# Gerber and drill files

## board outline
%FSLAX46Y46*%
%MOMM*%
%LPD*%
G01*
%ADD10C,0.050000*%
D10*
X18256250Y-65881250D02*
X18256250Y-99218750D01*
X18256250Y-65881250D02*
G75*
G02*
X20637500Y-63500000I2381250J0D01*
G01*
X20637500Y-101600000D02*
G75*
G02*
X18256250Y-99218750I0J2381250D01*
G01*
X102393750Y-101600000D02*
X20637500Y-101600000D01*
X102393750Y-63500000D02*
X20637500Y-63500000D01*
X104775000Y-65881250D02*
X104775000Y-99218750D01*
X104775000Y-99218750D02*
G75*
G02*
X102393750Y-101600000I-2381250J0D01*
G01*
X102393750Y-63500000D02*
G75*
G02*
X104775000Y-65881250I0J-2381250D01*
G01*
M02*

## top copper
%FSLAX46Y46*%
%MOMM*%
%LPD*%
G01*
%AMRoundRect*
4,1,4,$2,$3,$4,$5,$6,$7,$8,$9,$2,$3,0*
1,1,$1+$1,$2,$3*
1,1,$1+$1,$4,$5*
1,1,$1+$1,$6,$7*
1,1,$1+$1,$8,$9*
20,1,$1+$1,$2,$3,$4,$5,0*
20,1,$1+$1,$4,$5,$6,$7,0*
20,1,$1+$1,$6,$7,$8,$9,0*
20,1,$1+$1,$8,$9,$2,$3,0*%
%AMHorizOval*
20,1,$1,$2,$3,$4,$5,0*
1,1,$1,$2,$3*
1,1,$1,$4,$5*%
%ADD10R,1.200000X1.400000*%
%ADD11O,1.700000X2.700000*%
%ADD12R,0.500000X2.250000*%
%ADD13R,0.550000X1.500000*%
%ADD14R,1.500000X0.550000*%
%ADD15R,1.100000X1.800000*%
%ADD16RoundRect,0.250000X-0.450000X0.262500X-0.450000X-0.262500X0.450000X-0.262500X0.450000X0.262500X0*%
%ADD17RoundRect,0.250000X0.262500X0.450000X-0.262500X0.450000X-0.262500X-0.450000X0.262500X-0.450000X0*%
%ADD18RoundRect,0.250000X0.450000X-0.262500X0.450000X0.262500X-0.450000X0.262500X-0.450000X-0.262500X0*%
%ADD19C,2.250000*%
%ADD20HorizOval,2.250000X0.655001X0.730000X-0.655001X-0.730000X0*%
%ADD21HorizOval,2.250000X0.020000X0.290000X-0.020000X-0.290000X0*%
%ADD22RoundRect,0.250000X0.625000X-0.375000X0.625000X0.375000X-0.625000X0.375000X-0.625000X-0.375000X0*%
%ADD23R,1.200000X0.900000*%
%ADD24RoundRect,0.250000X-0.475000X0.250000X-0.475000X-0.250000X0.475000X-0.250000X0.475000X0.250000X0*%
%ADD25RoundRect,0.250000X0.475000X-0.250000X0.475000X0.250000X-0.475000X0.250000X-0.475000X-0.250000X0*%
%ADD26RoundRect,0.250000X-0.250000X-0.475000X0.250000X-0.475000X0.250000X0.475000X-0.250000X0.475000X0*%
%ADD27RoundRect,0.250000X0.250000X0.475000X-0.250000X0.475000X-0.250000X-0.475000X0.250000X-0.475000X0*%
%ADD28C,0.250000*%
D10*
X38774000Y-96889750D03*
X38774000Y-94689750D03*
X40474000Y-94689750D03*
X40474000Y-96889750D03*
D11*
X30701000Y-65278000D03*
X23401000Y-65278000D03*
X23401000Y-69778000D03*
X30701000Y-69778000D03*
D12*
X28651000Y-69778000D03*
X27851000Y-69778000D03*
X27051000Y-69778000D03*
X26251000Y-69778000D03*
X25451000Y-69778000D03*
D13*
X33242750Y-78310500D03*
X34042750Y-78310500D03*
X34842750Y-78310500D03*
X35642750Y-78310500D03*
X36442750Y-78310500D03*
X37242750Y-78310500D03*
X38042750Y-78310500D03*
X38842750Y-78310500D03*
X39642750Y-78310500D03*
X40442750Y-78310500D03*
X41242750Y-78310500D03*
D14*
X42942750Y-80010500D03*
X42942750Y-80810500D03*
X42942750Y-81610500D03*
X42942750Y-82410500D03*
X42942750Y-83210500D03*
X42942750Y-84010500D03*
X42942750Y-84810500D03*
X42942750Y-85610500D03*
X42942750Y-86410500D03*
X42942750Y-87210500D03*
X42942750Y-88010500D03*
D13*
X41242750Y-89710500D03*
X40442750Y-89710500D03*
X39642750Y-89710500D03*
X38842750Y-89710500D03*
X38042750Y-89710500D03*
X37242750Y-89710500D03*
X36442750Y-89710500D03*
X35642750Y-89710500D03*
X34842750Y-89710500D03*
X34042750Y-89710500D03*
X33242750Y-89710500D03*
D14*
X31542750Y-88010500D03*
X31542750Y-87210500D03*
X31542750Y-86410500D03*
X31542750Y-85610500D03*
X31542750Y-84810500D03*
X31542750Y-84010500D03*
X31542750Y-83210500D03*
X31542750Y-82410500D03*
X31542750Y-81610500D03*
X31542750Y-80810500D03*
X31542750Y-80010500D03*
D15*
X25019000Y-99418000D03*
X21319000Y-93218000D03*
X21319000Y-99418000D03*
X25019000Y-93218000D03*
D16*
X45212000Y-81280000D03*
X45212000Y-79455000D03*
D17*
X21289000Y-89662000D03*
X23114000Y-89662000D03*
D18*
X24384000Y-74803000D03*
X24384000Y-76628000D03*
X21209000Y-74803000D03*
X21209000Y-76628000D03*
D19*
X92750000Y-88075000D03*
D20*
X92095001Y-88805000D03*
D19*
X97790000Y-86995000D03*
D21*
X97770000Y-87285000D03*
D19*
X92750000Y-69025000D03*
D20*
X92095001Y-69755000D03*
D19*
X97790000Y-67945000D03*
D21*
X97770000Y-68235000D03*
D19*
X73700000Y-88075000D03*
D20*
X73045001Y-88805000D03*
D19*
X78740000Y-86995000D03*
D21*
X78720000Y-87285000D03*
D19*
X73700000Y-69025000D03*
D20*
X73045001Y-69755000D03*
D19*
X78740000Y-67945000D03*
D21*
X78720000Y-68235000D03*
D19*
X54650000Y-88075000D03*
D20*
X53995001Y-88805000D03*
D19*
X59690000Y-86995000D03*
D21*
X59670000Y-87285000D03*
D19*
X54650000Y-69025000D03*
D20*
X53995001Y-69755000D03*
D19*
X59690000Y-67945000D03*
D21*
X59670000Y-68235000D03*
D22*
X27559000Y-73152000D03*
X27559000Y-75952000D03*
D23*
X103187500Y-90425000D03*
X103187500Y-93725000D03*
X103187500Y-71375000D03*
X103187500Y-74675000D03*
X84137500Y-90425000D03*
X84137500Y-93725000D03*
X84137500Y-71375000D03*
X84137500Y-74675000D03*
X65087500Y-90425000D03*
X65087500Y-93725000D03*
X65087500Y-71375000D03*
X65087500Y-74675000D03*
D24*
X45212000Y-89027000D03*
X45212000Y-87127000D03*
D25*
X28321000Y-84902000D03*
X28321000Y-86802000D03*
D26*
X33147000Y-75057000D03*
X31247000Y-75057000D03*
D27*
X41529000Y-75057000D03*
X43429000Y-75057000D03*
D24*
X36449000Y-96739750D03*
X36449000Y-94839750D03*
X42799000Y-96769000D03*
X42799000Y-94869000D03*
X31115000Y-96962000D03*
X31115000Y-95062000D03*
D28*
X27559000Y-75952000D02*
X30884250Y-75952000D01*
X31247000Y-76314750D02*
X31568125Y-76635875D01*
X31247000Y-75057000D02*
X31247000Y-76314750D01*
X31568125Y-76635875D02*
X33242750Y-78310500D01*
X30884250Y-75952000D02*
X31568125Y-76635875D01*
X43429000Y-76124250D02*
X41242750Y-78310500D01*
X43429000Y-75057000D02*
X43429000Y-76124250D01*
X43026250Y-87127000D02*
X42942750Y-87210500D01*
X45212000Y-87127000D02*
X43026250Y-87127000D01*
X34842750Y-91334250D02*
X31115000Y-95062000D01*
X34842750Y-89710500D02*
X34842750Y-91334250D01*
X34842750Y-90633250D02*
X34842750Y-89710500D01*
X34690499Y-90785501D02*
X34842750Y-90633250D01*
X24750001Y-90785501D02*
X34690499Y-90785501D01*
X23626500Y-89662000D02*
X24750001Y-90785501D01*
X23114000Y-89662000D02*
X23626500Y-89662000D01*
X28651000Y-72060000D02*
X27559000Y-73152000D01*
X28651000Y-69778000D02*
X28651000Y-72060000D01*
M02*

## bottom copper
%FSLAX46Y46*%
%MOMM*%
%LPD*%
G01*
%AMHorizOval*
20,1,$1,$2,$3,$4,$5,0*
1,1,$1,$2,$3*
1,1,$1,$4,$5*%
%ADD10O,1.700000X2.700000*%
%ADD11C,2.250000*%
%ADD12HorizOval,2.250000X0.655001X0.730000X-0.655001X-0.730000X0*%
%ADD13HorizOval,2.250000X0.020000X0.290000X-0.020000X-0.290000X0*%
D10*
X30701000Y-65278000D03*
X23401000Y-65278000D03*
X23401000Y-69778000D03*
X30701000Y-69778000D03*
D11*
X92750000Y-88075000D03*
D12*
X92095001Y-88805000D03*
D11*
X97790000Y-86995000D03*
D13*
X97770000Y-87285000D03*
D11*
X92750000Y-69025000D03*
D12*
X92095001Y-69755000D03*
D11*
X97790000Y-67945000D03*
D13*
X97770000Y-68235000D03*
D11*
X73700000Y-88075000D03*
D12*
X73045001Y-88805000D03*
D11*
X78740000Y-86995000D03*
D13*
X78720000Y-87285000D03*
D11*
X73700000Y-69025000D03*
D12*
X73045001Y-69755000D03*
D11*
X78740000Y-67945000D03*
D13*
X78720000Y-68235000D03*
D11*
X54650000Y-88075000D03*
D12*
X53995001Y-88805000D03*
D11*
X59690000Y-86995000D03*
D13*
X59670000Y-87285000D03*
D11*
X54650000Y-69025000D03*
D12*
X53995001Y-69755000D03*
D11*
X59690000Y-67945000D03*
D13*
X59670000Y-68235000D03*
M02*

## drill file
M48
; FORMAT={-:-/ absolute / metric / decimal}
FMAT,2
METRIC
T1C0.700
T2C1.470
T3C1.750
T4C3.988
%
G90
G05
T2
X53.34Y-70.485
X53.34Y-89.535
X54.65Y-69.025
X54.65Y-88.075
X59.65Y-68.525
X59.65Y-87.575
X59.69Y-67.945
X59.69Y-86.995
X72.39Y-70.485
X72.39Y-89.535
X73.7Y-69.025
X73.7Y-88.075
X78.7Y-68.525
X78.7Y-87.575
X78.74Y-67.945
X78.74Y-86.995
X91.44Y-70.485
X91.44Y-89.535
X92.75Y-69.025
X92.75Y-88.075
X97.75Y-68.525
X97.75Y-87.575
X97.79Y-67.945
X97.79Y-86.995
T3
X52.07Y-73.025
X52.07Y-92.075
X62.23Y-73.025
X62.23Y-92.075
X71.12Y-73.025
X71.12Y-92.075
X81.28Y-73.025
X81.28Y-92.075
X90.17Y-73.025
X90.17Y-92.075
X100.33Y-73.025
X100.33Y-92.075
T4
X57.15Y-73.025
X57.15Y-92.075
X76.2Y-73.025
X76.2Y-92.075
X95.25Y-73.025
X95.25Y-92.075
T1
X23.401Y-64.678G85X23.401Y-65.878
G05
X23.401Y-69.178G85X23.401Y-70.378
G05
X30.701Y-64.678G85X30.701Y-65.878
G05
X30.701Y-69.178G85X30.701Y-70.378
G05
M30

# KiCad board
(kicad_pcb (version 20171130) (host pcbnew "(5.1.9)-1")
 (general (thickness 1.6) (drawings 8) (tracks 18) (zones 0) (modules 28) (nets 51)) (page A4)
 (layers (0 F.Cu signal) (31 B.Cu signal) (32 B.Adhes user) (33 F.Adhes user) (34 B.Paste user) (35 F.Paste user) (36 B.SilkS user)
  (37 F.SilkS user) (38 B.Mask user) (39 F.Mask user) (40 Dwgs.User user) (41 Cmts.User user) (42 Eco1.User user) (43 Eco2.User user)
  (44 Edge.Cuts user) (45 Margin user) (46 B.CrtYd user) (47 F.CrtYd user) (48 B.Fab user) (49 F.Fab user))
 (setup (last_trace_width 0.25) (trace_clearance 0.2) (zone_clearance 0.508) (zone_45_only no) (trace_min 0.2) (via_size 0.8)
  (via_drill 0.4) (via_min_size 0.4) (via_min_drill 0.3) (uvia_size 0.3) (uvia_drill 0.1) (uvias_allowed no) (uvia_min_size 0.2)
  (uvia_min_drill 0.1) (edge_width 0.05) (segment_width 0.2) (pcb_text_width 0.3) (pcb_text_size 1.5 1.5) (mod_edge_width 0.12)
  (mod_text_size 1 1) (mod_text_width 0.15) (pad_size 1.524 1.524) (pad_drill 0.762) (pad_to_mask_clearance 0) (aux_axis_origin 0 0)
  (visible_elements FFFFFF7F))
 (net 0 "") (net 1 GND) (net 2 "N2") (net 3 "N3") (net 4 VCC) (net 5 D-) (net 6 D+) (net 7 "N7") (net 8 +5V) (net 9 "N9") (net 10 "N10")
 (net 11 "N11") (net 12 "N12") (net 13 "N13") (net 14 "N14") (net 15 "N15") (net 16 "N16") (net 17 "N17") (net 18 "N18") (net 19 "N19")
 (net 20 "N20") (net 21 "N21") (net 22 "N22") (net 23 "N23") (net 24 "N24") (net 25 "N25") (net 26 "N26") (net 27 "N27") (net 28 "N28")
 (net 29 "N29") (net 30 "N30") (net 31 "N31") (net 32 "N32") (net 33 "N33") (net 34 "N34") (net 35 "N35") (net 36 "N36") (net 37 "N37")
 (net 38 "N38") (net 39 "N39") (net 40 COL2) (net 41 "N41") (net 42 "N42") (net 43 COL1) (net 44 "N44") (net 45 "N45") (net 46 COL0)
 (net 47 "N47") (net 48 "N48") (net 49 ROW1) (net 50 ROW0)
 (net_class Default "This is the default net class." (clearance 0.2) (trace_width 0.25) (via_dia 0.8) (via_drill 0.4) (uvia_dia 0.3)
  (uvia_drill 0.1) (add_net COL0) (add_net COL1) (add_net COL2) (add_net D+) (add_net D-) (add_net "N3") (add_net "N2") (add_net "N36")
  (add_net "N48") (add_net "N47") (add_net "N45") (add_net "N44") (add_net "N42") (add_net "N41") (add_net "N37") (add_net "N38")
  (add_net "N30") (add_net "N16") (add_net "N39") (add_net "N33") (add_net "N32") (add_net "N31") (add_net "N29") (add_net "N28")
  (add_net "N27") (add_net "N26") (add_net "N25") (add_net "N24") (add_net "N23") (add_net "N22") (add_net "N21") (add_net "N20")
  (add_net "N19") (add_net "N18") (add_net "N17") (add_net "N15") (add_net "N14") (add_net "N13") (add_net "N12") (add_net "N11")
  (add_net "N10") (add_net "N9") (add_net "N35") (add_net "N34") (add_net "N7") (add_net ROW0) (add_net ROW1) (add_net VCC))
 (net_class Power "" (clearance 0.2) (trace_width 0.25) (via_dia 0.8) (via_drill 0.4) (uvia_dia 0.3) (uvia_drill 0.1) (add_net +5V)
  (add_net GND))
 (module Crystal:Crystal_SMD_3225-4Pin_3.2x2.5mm (layer F.Cu) (at 39.624 95.78975 90)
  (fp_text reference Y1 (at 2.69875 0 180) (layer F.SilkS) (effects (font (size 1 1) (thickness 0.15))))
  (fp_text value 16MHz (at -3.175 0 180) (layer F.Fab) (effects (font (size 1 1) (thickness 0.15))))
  (pad 4 smd rect (at -1.1 -0.85 90) (size 1.4 1.2) (layers F.Cu F.Paste F.Mask) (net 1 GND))
  (pad 3 smd rect (at 1.1 -0.85 90) (size 1.4 1.2) (layers F.Cu F.Paste F.Mask) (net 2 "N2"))
  (pad 2 smd rect (at 1.1 0.85 90) (size 1.4 1.2) (layers F.Cu F.Paste F.Mask) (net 1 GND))
  (pad 1 smd rect (at -1.1 0.85 90) (size 1.4 1.2) (layers F.Cu F.Paste F.Mask) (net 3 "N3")))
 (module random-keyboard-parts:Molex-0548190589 (layer F.Cu) (at 27.051 65.278 270)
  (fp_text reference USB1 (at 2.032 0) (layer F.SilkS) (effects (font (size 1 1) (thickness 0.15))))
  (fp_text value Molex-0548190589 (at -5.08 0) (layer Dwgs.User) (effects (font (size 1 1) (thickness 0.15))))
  (pad 6 thru_hole oval (at 0 -3.65 270) (size 2.7 1.7) (drill oval 1.9 0.7) (layers *.Cu *.Mask) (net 1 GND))
  (pad 6 thru_hole oval (at 0 3.65 270) (size 2.7 1.7) (drill oval 1.9 0.7) (layers *.Cu *.Mask) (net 1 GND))
  (pad 6 thru_hole oval (at 4.5 3.65 270) (size 2.7 1.7) (drill oval 1.9 0.7) (layers *.Cu *.Mask) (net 1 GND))
  (pad 6 thru_hole oval (at 4.5 -3.65 270) (size 2.7 1.7) (drill oval 1.9 0.7) (layers *.Cu *.Mask) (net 1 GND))
  (pad 5 smd rect (at 4.5 -1.6 270) (size 2.25 0.5) (layers F.Cu F.Paste F.Mask) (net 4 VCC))
  (pad 4 smd rect (at 4.5 -0.8 270) (size 2.25 0.5) (layers F.Cu F.Paste F.Mask) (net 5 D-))
  (pad 3 smd rect (at 4.5 0 270) (size 2.25 0.5) (layers F.Cu F.Paste F.Mask) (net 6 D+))
  (pad 2 smd rect (at 4.5 0.8 270) (size 2.25 0.5) (layers F.Cu F.Paste F.Mask) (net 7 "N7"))
  (pad 1 smd rect (at 4.5 1.6 270) (size 2.25 0.5) (layers F.Cu F.Paste F.Mask) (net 1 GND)))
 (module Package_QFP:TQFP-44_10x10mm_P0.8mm (layer F.Cu) (at 37.24275 84.0105)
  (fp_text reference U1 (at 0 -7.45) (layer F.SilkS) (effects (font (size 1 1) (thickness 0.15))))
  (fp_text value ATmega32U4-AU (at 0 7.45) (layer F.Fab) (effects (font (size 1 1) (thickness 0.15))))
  (pad 44 smd rect (at -4 -5.7 90) (size 1.5 0.55) (layers F.Cu F.Paste F.Mask) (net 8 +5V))
  (pad 43 smd rect (at -3.2 -5.7 90) (size 1.5 0.55) (layers F.Cu F.Paste F.Mask) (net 1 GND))
  (pad 42 smd rect (at -2.4 -5.7 90) (size 1.5 0.55) (layers F.Cu F.Paste F.Mask) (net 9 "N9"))
  (pad 41 smd rect (at -1.6 -5.7 90) (size 1.5 0.55) (layers F.Cu F.Paste F.Mask) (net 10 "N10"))
  (pad 40 smd rect (at -0.8 -5.7 90) (size 1.5 0.55) (layers F.Cu F.Paste F.Mask) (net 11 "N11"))
  (pad 39 smd rect (at 0 -5.7 90) (size 1.5 0.55) (layers F.Cu F.Paste F.Mask) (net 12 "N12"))
  (pad 38 smd rect (at 0.8 -5.7 90) (size 1.5 0.55) (layers F.Cu F.Paste F.Mask) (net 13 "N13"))
  (pad 37 smd rect (at 1.6 -5.7 90) (size 1.5 0.55) (layers F.Cu F.Paste F.Mask) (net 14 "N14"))
  (pad 36 smd rect (at 2.4 -5.7 90) (size 1.5 0.55) (layers F.Cu F.Paste F.Mask) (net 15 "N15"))
  (pad 35 smd rect (at 3.2 -5.7 90) (size 1.5 0.55) (layers F.Cu F.Paste F.Mask) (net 1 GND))
  (pad 34 smd rect (at 4 -5.7 90) (size 1.5 0.55) (layers F.Cu F.Paste F.Mask) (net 8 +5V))
  (pad 33 smd rect (at 5.7 -4) (size 1.5 0.55) (layers F.Cu F.Paste F.Mask) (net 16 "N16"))
  (pad 32 smd rect (at 5.7 -3.2) (size 1.5 0.55) (layers F.Cu F.Paste F.Mask) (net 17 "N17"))
  (pad 31 smd rect (at 5.7 -2.4) (size 1.5 0.55) (layers F.Cu F.Paste F.Mask) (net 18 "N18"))
  (pad 30 smd rect (at 5.7 -1.6) (size 1.5 0.55) (layers F.Cu F.Paste F.Mask) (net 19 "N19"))
  (pad 29 smd rect (at 5.7 -0.8) (size 1.5 0.55) (layers F.Cu F.Paste F.Mask) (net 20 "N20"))
  (pad 28 smd rect (at 5.7 0) (size 1.5 0.55) (layers F.Cu F.Paste F.Mask) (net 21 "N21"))
  (pad 27 smd rect (at 5.7 0.8) (size 1.5 0.55) (layers F.Cu F.Paste F.Mask) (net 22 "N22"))
  (pad 26 smd rect (at 5.7 1.6) (size 1.5 0.55) (layers F.Cu F.Paste F.Mask) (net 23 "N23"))
  (pad 25 smd rect (at 5.7 2.4) (size 1.5 0.55) (layers F.Cu F.Paste F.Mask) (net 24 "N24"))
  (pad 24 smd rect (at 5.7 3.2) (size 1.5 0.55) (layers F.Cu F.Paste F.Mask) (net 8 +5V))
  (pad 23 smd rect (at 5.7 4) (size 1.5 0.55) (layers F.Cu F.Paste F.Mask) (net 1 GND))
  (pad 22 smd rect (at 4 5.7 90) (size 1.5 0.55) (layers F.Cu F.Paste F.Mask) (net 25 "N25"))
  (pad 21 smd rect (at 3.2 5.7 90) (size 1.5 0.55) (layers F.Cu F.Paste F.Mask) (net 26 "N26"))
  (pad 20 smd rect (at 2.4 5.7 90) (size 1.5 0.55) (layers F.Cu F.Paste F.Mask) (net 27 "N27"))
  (pad 19 smd rect (at 1.6 5.7 90) (size 1.5 0.55) (layers F.Cu F.Paste F.Mask) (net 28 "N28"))
  (pad 18 smd rect (at 0.8 5.7 90) (size 1.5 0.55) (layers F.Cu F.Paste F.Mask) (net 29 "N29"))
  (pad 17 smd rect (at 0 5.7 90) (size 1.5 0.55) (layers F.Cu F.Paste F.Mask) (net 3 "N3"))
  (pad 16 smd rect (at -0.8 5.7 90) (size 1.5 0.55) (layers F.Cu F.Paste F.Mask) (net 2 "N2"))
  (pad 15 smd rect (at -1.6 5.7 90) (size 1.5 0.55) (layers F.Cu F.Paste F.Mask) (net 1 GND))
  (pad 14 smd rect (at -2.4 5.7 90) (size 1.5 0.55) (layers F.Cu F.Paste F.Mask) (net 8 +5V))
  (pad 13 smd rect (at -3.2 5.7 90) (size 1.5 0.55) (layers F.Cu F.Paste F.Mask) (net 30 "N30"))
  (pad 12 smd rect (at -4 5.7 90) (size 1.5 0.55) (layers F.Cu F.Paste F.Mask) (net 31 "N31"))
  (pad 11 smd rect (at -5.7 4) (size 1.5 0.55) (layers F.Cu F.Paste F.Mask) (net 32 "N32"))
  (pad 10 smd rect (at -5.7 3.2) (size 1.5 0.55) (layers F.Cu F.Paste F.Mask) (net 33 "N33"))
  (pad 9 smd rect (at -5.7 2.4) (size 1.5 0.55) (layers F.Cu F.Paste F.Mask) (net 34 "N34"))
  (pad 8 smd rect (at -5.7 1.6) (size 1.5 0.55) (layers F.Cu F.Paste F.Mask) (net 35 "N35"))
  (pad 7 smd rect (at -5.7 0.8) (size 1.5 0.55) (layers F.Cu F.Paste F.Mask) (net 8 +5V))
  (pad 6 smd rect (at -5.7 0) (size 1.5 0.55) (layers F.Cu F.Paste F.Mask) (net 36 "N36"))
  (pad 5 smd rect (at -5.7 -0.8) (size 1.5 0.55) (layers F.Cu F.Paste F.Mask) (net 1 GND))
  (pad 4 smd rect (at -5.7 -1.6) (size 1.5 0.55) (layers F.Cu F.Paste F.Mask) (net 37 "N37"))
  (pad 3 smd rect (at -5.7 -2.4) (size 1.5 0.55) (layers F.Cu F.Paste F.Mask) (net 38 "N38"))
  (pad 2 smd rect (at -5.7 -3.2) (size 1.5 0.55) (layers F.Cu F.Paste F.Mask) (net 8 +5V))
  (pad 1 smd rect (at -5.7 -4) (size 1.5 0.55) (layers F.Cu F.Paste F.Mask) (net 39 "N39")))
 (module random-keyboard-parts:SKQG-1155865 (layer F.Cu) (at 23.169 96.318 90)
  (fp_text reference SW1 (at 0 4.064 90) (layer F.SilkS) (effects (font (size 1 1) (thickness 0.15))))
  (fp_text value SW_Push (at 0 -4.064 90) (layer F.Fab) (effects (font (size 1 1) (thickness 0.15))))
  (pad 4 smd rect (at -3.1 1.85 90) (size 1.8 1.1) (layers F.Cu F.Paste F.Mask))
  (pad 3 smd rect (at 3.1 -1.85 90) (size 1.8 1.1) (layers F.Cu F.Paste F.Mask))
  (pad 2 smd rect (at -3.1 -1.85 90) (size 1.8 1.1) (layers F.Cu F.Paste F.Mask) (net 30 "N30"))
  (pad 1 smd rect (at 3.1 1.85 90) (size 1.8 1.1) (layers F.Cu F.Paste F.Mask) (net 1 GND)))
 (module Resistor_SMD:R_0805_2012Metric (layer F.Cu) (at 45.212 80.3675 270)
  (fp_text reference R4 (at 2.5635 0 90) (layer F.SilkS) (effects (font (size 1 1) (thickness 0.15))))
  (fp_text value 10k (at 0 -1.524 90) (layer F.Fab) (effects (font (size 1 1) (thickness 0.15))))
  (pad 2 smd roundrect (at 0.9125 0 270) (size 1.025 1.4) (layers F.Cu F.Paste F.Mask) (roundrect_rratio 0.243902) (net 16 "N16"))
  (pad 1 smd roundrect (at -0.9125 0 270) (size 1.025 1.4) (layers F.Cu F.Paste F.Mask) (roundrect_rratio 0.243902) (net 1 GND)))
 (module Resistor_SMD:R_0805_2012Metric (layer F.Cu) (at 22.2015 89.662 180)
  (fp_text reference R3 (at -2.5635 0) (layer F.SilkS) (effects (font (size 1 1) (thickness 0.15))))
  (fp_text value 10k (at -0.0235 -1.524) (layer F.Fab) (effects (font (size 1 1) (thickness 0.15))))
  (pad 2 smd roundrect (at 0.9125 0 180) (size 1.025 1.4) (layers F.Cu F.Paste F.Mask) (roundrect_rratio 0.243902) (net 30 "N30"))
  (pad 1 smd roundrect (at -0.9125 0 180) (size 1.025 1.4) (layers F.Cu F.Paste F.Mask) (roundrect_rratio 0.243902) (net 8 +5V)))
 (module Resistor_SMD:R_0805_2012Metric (layer F.Cu) (at 24.384 75.7155 90)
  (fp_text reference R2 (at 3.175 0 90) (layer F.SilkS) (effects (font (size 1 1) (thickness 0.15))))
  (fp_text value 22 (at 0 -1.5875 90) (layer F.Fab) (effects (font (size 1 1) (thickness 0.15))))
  (pad 2 smd roundrect (at 0.9125 0 90) (size 1.025 1.4) (layers F.Cu F.Paste F.Mask) (roundrect_rratio 0.243902) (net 5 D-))
  (pad 1 smd roundrect (at -0.9125 0 90) (size 1.025 1.4) (layers F.Cu F.Paste F.Mask) (roundrect_rratio 0.243902) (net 38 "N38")))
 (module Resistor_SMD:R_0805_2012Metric (layer F.Cu) (at 21.209 75.7155 90)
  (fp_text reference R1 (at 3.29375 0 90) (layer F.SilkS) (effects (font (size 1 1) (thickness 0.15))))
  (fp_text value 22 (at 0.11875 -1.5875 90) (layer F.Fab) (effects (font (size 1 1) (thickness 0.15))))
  (pad 2 smd roundrect (at 0.9125 0 90) (size 1.025 1.4) (layers F.Cu F.Paste F.Mask) (roundrect_rratio 0.243902) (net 6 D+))
  (pad 1 smd roundrect (at -0.9125 0 90) (size 1.025 1.4) (layers F.Cu F.Paste F.Mask) (roundrect_rratio 0.243902) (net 37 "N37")))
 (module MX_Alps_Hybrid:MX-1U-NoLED (layer F.Cu) (at 95.25 92.075)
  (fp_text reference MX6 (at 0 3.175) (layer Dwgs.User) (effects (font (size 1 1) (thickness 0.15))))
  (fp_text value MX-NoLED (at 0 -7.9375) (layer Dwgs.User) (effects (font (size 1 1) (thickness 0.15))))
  (pad "" np_thru_hole circle (at 5.08 0 48.0996) (size 1.75 1.75) (drill 1.75) (layers *.Cu *.Mask))
  (pad "" np_thru_hole circle (at -5.08 0 48.0996) (size 1.75 1.75) (drill 1.75) (layers *.Cu *.Mask))
  (pad 1 thru_hole circle (at -2.5 -4) (size 2.25 2.25) (drill 1.47) (layers *.Cu B.Mask) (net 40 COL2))
  (pad "" np_thru_hole circle (at 0 0) (size 3.9878 3.9878) (drill 3.9878) (layers *.Cu *.Mask))
  (pad 1 thru_hole oval (at -3.81 -2.54 48.0996) (size 4.211556 2.25) (drill 1.47 (offset 0.980778 0)) (layers *.Cu B.Mask) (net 40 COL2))
  (pad 2 thru_hole circle (at 2.54 -5.08) (size 2.25 2.25) (drill 1.47) (layers *.Cu B.Mask) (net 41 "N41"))
  (pad 2 thru_hole oval (at 2.5 -4.5 86.0548) (size 2.831378 2.25) (drill 1.47 (offset 0.290689 0)) (layers *.Cu B.Mask) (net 41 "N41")))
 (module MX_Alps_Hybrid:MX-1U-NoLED (layer F.Cu) (at 95.25 73.025)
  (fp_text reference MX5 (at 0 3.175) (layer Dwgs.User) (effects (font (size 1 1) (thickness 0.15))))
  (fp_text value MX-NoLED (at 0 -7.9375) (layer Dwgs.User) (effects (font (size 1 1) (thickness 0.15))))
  (pad "" np_thru_hole circle (at 5.08 0 48.0996) (size 1.75 1.75) (drill 1.75) (layers *.Cu *.Mask))
  (pad "" np_thru_hole circle (at -5.08 0 48.0996) (size 1.75 1.75) (drill 1.75) (layers *.Cu *.Mask))
  (pad 1 thru_hole circle (at -2.5 -4) (size 2.25 2.25) (drill 1.47) (layers *.Cu B.Mask) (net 40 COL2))
  (pad "" np_thru_hole circle (at 0 0) (size 3.9878 3.9878) (drill 3.9878) (layers *.Cu *.Mask))
  (pad 1 thru_hole oval (at -3.81 -2.54 48.0996) (size 4.211556 2.25) (drill 1.47 (offset 0.980778 0)) (layers *.Cu B.Mask) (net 40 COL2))
  (pad 2 thru_hole circle (at 2.54 -5.08) (size 2.25 2.25) (drill 1.47) (layers *.Cu B.Mask) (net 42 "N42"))
  (pad 2 thru_hole oval (at 2.5 -4.5 86.0548) (size 2.831378 2.25) (drill 1.47 (offset 0.290689 0)) (layers *.Cu B.Mask) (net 42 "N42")))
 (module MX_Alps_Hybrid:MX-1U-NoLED (layer F.Cu) (at 76.2 92.075)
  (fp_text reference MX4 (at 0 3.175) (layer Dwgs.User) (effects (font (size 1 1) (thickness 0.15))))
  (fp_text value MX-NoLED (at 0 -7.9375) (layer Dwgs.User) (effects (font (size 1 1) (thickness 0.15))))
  (pad "" np_thru_hole circle (at 5.08 0 48.0996) (size 1.75 1.75) (drill 1.75) (layers *.Cu *.Mask))
  (pad "" np_thru_hole circle (at -5.08 0 48.0996) (size 1.75 1.75) (drill 1.75) (layers *.Cu *.Mask))
  (pad 1 thru_hole circle (at -2.5 -4) (size 2.25 2.25) (drill 1.47) (layers *.Cu B.Mask) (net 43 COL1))
  (pad "" np_thru_hole circle (at 0 0) (size 3.9878 3.9878) (drill 3.9878) (layers *.Cu *.Mask))
  (pad 1 thru_hole oval (at -3.81 -2.54 48.0996) (size 4.211556 2.25) (drill 1.47 (offset 0.980778 0)) (layers *.Cu B.Mask) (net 43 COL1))
  (pad 2 thru_hole circle (at 2.54 -5.08) (size 2.25 2.25) (drill 1.47) (layers *.Cu B.Mask) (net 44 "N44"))
  (pad 2 thru_hole oval (at 2.5 -4.5 86.0548) (size 2.831378 2.25) (drill 1.47 (offset 0.290689 0)) (layers *.Cu B.Mask) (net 44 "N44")))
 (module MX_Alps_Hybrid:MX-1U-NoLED (layer F.Cu) (at 76.2 73.025)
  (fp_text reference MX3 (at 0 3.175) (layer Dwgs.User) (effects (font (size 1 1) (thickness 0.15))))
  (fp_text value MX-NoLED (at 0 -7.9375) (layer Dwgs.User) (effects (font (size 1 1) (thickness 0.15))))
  (pad "" np_thru_hole circle (at 5.08 0 48.0996) (size 1.75 1.75) (drill 1.75) (layers *.Cu *.Mask))
  (pad "" np_thru_hole circle (at -5.08 0 48.0996) (size 1.75 1.75) (drill 1.75) (layers *.Cu *.Mask))
  (pad 1 thru_hole circle (at -2.5 -4) (size 2.25 2.25) (drill 1.47) (layers *.Cu B.Mask) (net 43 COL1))
  (pad "" np_thru_hole circle (at 0 0) (size 3.9878 3.9878) (drill 3.9878) (layers *.Cu *.Mask))
  (pad 1 thru_hole oval (at -3.81 -2.54 48.0996) (size 4.211556 2.25) (drill 1.47 (offset 0.980778 0)) (layers *.Cu B.Mask) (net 43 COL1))
  (pad 2 thru_hole circle (at 2.54 -5.08) (size 2.25 2.25) (drill 1.47) (layers *.Cu B.Mask) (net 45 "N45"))
  (pad 2 thru_hole oval (at 2.5 -4.5 86.0548) (size 2.831378 2.25) (drill 1.47 (offset 0.290689 0)) (layers *.Cu B.Mask) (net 45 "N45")))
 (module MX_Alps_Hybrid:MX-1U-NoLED (layer F.Cu) (at 57.15 92.075)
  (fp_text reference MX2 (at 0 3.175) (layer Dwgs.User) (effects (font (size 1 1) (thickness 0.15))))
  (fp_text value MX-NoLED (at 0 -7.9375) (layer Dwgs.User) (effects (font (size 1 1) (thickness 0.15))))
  (pad "" np_thru_hole circle (at 5.08 0 48.0996) (size 1.75 1.75) (drill 1.75) (layers *.Cu *.Mask))
  (pad "" np_thru_hole circle (at -5.08 0 48.0996) (size 1.75 1.75) (drill 1.75) (layers *.Cu *.Mask))
  (pad 1 thru_hole circle (at -2.5 -4) (size 2.25 2.25) (drill 1.47) (layers *.Cu B.Mask) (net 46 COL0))
  (pad "" np_thru_hole circle (at 0 0) (size 3.9878 3.9878) (drill 3.9878) (layers *.Cu *.Mask))
  (pad 1 thru_hole oval (at -3.81 -2.54 48.0996) (size 4.211556 2.25) (drill 1.47 (offset 0.980778 0)) (layers *.Cu B.Mask) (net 46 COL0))
  (pad 2 thru_hole circle (at 2.54 -5.08) (size 2.25 2.25) (drill 1.47) (layers *.Cu B.Mask) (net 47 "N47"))
  (pad 2 thru_hole oval (at 2.5 -4.5 86.0548) (size 2.831378 2.25) (drill 1.47 (offset 0.290689 0)) (layers *.Cu B.Mask) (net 47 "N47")))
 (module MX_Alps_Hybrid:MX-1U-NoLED (layer F.Cu) (at 57.15 73.025)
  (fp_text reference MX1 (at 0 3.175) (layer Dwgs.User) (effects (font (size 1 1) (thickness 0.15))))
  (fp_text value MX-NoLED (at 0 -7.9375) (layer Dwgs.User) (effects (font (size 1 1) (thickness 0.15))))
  (pad "" np_thru_hole circle (at 5.08 0 48.0996) (size 1.75 1.75) (drill 1.75) (layers *.Cu *.Mask))
  (pad "" np_thru_hole circle (at -5.08 0 48.0996) (size 1.75 1.75) (drill 1.75) (layers *.Cu *.Mask))
  (pad 1 thru_hole circle (at -2.5 -4) (size 2.25 2.25) (drill 1.47) (layers *.Cu B.Mask) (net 46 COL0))
  (pad "" np_thru_hole circle (at 0 0) (size 3.9878 3.9878) (drill 3.9878) (layers *.Cu *.Mask))
  (pad 1 thru_hole oval (at -3.81 -2.54 48.0996) (size 4.211556 2.25) (drill 1.47 (offset 0.980778 0)) (layers *.Cu B.Mask) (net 46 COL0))
  (pad 2 thru_hole circle (at 2.54 -5.08) (size 2.25 2.25) (drill 1.47) (layers *.Cu B.Mask) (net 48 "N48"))
  (pad 2 thru_hole oval (at 2.5 -4.5 86.0548) (size 2.831378 2.25) (drill 1.47 (offset 0.290689 0)) (layers *.Cu B.Mask) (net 48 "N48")))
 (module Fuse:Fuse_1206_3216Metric (layer F.Cu) (at 27.559 74.552 90)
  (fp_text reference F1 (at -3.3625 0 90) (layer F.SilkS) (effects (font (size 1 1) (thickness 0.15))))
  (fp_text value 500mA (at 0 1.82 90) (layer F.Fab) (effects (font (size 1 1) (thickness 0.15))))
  (pad 2 smd roundrect (at 1.4 0 90) (size 1.25 1.75) (layers F.Cu F.Paste F.Mask) (roundrect_rratio 0.2) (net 4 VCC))
  (pad 1 smd roundrect (at -1.4 0 90) (size 1.25 1.75) (layers F.Cu F.Paste F.Mask) (roundrect_rratio 0.2) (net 8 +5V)))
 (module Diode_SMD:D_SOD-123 (layer F.Cu) (at 103.1875 92.075 90)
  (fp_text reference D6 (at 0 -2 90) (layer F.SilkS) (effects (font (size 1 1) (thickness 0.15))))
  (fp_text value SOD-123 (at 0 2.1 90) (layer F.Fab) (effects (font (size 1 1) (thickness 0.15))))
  (pad 2 smd rect (at 1.65 0 90) (size 0.9 1.2) (layers F.Cu F.Paste F.Mask) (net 41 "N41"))
  (pad 1 smd rect (at -1.65 0 90) (size 0.9 1.2) (layers F.Cu F.Paste F.Mask) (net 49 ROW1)))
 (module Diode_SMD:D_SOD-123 (layer F.Cu) (at 103.1875 73.025 90)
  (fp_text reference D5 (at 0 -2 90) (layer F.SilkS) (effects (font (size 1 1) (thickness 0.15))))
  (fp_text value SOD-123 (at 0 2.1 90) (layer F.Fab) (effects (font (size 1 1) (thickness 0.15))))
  (pad 2 smd rect (at 1.65 0 90) (size 0.9 1.2) (layers F.Cu F.Paste F.Mask) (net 42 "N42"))
  (pad 1 smd rect (at -1.65 0 90) (size 0.9 1.2) (layers F.Cu F.Paste F.Mask) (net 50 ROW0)))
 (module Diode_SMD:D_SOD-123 (layer F.Cu) (at 84.1375 92.075 90)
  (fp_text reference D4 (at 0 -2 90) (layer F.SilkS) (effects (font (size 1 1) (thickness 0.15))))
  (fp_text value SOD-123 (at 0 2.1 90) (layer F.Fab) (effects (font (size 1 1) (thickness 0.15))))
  (pad 2 smd rect (at 1.65 0 90) (size 0.9 1.2) (layers F.Cu F.Paste F.Mask) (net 44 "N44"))
  (pad 1 smd rect (at -1.65 0 90) (size 0.9 1.2) (layers F.Cu F.Paste F.Mask) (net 49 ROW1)))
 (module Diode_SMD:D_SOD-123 (layer F.Cu) (at 84.1375 73.025 90)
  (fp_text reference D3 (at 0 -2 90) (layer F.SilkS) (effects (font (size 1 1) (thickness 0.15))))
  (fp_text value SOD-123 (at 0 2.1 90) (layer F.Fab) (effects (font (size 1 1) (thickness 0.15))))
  (pad 2 smd rect (at 1.65 0 90) (size 0.9 1.2) (layers F.Cu F.Paste F.Mask) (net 45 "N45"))
  (pad 1 smd rect (at -1.65 0 90) (size 0.9 1.2) (layers F.Cu F.Paste F.Mask) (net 50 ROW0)))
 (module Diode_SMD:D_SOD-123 (layer F.Cu) (at 65.0875 92.075 90)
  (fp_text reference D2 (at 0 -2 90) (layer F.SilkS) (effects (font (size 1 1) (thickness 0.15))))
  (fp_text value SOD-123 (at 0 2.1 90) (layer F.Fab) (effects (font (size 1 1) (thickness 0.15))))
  (pad 2 smd rect (at 1.65 0 90) (size 0.9 1.2) (layers F.Cu F.Paste F.Mask) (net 47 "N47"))
  (pad 1 smd rect (at -1.65 0 90) (size 0.9 1.2) (layers F.Cu F.Paste F.Mask) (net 49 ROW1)))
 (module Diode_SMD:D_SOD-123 (layer F.Cu) (at 65.0875 73.025 90)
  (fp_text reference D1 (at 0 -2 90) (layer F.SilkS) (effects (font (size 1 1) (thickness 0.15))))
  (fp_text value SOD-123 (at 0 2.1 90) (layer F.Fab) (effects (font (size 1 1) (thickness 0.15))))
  (pad 2 smd rect (at 1.65 0 90) (size 0.9 1.2) (layers F.Cu F.Paste F.Mask) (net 48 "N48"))
  (pad 1 smd rect (at -1.65 0 90) (size 0.9 1.2) (layers F.Cu F.Paste F.Mask) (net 50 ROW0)))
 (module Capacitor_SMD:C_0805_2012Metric (layer F.Cu) (at 45.212 88.077 270)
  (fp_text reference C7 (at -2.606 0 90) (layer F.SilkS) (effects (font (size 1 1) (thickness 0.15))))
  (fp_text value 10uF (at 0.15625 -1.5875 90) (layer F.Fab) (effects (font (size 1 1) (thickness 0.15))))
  (pad 2 smd roundrect (at 0.95 0 270) (size 1 1.45) (layers F.Cu F.Paste F.Mask) (roundrect_rratio 0.25) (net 1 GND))
  (pad 1 smd roundrect (at -0.95 0 270) (size 1 1.45) (layers F.Cu F.Paste F.Mask) (roundrect_rratio 0.25) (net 8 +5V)))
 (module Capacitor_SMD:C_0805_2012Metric (layer F.Cu) (at 28.321 85.852 90)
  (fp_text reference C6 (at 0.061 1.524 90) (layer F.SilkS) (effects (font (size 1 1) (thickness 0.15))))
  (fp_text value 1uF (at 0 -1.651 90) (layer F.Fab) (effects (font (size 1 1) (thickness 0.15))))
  (pad 2 smd roundrect (at 0.95 0 90) (size 1 1.45) (layers F.Cu F.Paste F.Mask) (roundrect_rratio 0.25) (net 1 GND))
  (pad 1 smd roundrect (at -0.95 0 90) (size 1 1.45) (layers F.Cu F.Paste F.Mask) (roundrect_rratio 0.25) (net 36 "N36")))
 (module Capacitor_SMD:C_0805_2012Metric (layer F.Cu) (at 32.197 75.057)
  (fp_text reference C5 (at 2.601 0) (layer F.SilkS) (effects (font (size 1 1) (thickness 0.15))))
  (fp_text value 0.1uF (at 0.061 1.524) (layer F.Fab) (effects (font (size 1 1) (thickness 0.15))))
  (pad 2 smd roundrect (at 0.95 0) (size 1 1.45) (layers F.Cu F.Paste F.Mask) (roundrect_rratio 0.25) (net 1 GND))
  (pad 1 smd roundrect (at -0.95 0) (size 1 1.45) (layers F.Cu F.Paste F.Mask) (roundrect_rratio 0.25) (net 8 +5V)))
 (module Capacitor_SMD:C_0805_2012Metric (layer F.Cu) (at 42.479 75.057 180)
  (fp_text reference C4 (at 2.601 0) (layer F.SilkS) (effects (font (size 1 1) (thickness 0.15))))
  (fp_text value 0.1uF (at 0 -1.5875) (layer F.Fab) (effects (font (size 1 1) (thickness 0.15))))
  (pad 2 smd roundrect (at 0.95 0 180) (size 1 1.45) (layers F.Cu F.Paste F.Mask) (roundrect_rratio 0.25) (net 1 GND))
  (pad 1 smd roundrect (at -0.95 0 180) (size 1 1.45) (layers F.Cu F.Paste F.Mask) (roundrect_rratio 0.25) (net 8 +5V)))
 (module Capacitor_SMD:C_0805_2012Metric (layer F.Cu) (at 36.449 95.78975 270)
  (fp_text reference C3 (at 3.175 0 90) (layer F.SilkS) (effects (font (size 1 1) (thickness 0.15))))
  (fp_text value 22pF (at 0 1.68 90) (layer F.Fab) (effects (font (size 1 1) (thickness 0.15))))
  (pad 2 smd roundrect (at 0.95 0 270) (size 1 1.45) (layers F.Cu F.Paste F.Mask) (roundrect_rratio 0.25) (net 1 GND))
  (pad 1 smd roundrect (at -0.95 0 270) (size 1 1.45) (layers F.Cu F.Paste F.Mask) (roundrect_rratio 0.25) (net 2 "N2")))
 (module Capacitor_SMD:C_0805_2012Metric (layer F.Cu) (at 42.799 95.819 270)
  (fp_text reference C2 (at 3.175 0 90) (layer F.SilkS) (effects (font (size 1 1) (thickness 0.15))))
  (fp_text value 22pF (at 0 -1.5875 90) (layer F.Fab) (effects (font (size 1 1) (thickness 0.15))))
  (pad 2 smd roundrect (at 0.95 0 270) (size 1 1.45) (layers F.Cu F.Paste F.Mask) (roundrect_rratio 0.25) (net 1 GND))
  (pad 1 smd roundrect (at -0.95 0 270) (size 1 1.45) (layers F.Cu F.Paste F.Mask) (roundrect_rratio 0.25) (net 3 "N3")))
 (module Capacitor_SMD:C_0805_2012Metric (layer F.Cu) (at 31.115 96.012 270)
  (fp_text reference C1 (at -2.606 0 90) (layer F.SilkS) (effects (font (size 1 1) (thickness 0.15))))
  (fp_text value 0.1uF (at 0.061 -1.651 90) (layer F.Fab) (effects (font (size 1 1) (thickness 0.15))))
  (pad 2 smd roundrect (at 0.95 0 270) (size 1 1.45) (layers F.Cu F.Paste F.Mask) (roundrect_rratio 0.25) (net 1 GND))
  (pad 1 smd roundrect (at -0.95 0 270) (size 1 1.45) (layers F.Cu F.Paste F.Mask) (roundrect_rratio 0.25) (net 8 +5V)))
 (gr_line (start 18.25625 65.88125) (end 18.25625 99.21875) (layer Edge.Cuts) (width 0.05))
 (gr_arc (start 20.6375 65.88125) (end 20.6375 63.5) (angle -90) (layer Edge.Cuts) (width 0.05))
 (gr_arc (start 20.6375 99.21875) (end 18.25625 99.21875) (angle -90) (layer Edge.Cuts) (width 0.05))
 (gr_line (start 102.39375 101.6) (end 20.6375 101.6) (layer Edge.Cuts) (width 0.05))
 (gr_line (start 102.39375 63.5) (end 20.6375 63.5) (layer Edge.Cuts) (width 0.05))
 (gr_line (start 104.775 65.88125) (end 104.775 99.21875) (layer Edge.Cuts) (width 0.05))
 (gr_arc (start 102.39375 99.21875) (end 102.39375 101.6) (angle -90) (layer Edge.Cuts) (width 0.05))
 (gr_arc (start 102.39375 65.88125) (end 104.775 65.88125) (angle -90) (layer Edge.Cuts) (width 0.05))
 (segment (start 27.559 75.952) (end 30.88425 75.952) (width 0.25) (layer F.Cu) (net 8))
 (segment (start 31.247 76.31475) (end 31.568125 76.635875) (width 0.25) (layer F.Cu) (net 8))
 (segment (start 31.247 75.057) (end 31.247 76.31475) (width 0.25) (layer F.Cu) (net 8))
 (segment (start 31.568125 76.635875) (end 33.24275 78.3105) (width 0.25) (layer F.Cu) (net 8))
 (segment (start 30.88425 75.952) (end 31.568125 76.635875) (width 0.25) (layer F.Cu) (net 8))
 (segment (start 43.429 76.12425) (end 41.24275 78.3105) (width 0.25) (layer F.Cu) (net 8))
 (segment (start 43.429 75.057) (end 43.429 76.12425) (width 0.25) (layer F.Cu) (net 8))
 (segment (start 43.02625 87.127) (end 42.94275 87.2105) (width 0.25) (layer F.Cu) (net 8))
 (segment (start 45.212 87.127) (end 43.02625 87.127) (width 0.25) (layer F.Cu) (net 8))
 (segment (start 34.84275 91.33425) (end 31.115 95.062) (width 0.25) (layer F.Cu) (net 8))
 (segment (start 34.84275 89.7105) (end 34.84275 91.33425) (width 0.25) (layer F.Cu) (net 8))
 (segment (start 34.84275 90.63325) (end 34.84275 89.7105) (width 0.25) (layer F.Cu) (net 8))
 (segment (start 34.690499 90.785501) (end 34.84275 90.63325) (width 0.25) (layer F.Cu) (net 8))
 (segment (start 24.750001 90.785501) (end 34.690499 90.785501) (width 0.25) (layer F.Cu) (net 8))
 (segment (start 23.6265 89.662) (end 24.750001 90.785501) (width 0.25) (layer F.Cu) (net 8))
 (segment (start 23.114 89.662) (end 23.6265 89.662) (width 0.25) (layer F.Cu) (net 8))
 (segment (start 28.651 72.06) (end 27.559 73.152) (width 0.25) (layer F.Cu) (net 4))
 (segment (start 28.651 69.778) (end 28.651 72.06) (width 0.25) (layer F.Cu) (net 4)))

